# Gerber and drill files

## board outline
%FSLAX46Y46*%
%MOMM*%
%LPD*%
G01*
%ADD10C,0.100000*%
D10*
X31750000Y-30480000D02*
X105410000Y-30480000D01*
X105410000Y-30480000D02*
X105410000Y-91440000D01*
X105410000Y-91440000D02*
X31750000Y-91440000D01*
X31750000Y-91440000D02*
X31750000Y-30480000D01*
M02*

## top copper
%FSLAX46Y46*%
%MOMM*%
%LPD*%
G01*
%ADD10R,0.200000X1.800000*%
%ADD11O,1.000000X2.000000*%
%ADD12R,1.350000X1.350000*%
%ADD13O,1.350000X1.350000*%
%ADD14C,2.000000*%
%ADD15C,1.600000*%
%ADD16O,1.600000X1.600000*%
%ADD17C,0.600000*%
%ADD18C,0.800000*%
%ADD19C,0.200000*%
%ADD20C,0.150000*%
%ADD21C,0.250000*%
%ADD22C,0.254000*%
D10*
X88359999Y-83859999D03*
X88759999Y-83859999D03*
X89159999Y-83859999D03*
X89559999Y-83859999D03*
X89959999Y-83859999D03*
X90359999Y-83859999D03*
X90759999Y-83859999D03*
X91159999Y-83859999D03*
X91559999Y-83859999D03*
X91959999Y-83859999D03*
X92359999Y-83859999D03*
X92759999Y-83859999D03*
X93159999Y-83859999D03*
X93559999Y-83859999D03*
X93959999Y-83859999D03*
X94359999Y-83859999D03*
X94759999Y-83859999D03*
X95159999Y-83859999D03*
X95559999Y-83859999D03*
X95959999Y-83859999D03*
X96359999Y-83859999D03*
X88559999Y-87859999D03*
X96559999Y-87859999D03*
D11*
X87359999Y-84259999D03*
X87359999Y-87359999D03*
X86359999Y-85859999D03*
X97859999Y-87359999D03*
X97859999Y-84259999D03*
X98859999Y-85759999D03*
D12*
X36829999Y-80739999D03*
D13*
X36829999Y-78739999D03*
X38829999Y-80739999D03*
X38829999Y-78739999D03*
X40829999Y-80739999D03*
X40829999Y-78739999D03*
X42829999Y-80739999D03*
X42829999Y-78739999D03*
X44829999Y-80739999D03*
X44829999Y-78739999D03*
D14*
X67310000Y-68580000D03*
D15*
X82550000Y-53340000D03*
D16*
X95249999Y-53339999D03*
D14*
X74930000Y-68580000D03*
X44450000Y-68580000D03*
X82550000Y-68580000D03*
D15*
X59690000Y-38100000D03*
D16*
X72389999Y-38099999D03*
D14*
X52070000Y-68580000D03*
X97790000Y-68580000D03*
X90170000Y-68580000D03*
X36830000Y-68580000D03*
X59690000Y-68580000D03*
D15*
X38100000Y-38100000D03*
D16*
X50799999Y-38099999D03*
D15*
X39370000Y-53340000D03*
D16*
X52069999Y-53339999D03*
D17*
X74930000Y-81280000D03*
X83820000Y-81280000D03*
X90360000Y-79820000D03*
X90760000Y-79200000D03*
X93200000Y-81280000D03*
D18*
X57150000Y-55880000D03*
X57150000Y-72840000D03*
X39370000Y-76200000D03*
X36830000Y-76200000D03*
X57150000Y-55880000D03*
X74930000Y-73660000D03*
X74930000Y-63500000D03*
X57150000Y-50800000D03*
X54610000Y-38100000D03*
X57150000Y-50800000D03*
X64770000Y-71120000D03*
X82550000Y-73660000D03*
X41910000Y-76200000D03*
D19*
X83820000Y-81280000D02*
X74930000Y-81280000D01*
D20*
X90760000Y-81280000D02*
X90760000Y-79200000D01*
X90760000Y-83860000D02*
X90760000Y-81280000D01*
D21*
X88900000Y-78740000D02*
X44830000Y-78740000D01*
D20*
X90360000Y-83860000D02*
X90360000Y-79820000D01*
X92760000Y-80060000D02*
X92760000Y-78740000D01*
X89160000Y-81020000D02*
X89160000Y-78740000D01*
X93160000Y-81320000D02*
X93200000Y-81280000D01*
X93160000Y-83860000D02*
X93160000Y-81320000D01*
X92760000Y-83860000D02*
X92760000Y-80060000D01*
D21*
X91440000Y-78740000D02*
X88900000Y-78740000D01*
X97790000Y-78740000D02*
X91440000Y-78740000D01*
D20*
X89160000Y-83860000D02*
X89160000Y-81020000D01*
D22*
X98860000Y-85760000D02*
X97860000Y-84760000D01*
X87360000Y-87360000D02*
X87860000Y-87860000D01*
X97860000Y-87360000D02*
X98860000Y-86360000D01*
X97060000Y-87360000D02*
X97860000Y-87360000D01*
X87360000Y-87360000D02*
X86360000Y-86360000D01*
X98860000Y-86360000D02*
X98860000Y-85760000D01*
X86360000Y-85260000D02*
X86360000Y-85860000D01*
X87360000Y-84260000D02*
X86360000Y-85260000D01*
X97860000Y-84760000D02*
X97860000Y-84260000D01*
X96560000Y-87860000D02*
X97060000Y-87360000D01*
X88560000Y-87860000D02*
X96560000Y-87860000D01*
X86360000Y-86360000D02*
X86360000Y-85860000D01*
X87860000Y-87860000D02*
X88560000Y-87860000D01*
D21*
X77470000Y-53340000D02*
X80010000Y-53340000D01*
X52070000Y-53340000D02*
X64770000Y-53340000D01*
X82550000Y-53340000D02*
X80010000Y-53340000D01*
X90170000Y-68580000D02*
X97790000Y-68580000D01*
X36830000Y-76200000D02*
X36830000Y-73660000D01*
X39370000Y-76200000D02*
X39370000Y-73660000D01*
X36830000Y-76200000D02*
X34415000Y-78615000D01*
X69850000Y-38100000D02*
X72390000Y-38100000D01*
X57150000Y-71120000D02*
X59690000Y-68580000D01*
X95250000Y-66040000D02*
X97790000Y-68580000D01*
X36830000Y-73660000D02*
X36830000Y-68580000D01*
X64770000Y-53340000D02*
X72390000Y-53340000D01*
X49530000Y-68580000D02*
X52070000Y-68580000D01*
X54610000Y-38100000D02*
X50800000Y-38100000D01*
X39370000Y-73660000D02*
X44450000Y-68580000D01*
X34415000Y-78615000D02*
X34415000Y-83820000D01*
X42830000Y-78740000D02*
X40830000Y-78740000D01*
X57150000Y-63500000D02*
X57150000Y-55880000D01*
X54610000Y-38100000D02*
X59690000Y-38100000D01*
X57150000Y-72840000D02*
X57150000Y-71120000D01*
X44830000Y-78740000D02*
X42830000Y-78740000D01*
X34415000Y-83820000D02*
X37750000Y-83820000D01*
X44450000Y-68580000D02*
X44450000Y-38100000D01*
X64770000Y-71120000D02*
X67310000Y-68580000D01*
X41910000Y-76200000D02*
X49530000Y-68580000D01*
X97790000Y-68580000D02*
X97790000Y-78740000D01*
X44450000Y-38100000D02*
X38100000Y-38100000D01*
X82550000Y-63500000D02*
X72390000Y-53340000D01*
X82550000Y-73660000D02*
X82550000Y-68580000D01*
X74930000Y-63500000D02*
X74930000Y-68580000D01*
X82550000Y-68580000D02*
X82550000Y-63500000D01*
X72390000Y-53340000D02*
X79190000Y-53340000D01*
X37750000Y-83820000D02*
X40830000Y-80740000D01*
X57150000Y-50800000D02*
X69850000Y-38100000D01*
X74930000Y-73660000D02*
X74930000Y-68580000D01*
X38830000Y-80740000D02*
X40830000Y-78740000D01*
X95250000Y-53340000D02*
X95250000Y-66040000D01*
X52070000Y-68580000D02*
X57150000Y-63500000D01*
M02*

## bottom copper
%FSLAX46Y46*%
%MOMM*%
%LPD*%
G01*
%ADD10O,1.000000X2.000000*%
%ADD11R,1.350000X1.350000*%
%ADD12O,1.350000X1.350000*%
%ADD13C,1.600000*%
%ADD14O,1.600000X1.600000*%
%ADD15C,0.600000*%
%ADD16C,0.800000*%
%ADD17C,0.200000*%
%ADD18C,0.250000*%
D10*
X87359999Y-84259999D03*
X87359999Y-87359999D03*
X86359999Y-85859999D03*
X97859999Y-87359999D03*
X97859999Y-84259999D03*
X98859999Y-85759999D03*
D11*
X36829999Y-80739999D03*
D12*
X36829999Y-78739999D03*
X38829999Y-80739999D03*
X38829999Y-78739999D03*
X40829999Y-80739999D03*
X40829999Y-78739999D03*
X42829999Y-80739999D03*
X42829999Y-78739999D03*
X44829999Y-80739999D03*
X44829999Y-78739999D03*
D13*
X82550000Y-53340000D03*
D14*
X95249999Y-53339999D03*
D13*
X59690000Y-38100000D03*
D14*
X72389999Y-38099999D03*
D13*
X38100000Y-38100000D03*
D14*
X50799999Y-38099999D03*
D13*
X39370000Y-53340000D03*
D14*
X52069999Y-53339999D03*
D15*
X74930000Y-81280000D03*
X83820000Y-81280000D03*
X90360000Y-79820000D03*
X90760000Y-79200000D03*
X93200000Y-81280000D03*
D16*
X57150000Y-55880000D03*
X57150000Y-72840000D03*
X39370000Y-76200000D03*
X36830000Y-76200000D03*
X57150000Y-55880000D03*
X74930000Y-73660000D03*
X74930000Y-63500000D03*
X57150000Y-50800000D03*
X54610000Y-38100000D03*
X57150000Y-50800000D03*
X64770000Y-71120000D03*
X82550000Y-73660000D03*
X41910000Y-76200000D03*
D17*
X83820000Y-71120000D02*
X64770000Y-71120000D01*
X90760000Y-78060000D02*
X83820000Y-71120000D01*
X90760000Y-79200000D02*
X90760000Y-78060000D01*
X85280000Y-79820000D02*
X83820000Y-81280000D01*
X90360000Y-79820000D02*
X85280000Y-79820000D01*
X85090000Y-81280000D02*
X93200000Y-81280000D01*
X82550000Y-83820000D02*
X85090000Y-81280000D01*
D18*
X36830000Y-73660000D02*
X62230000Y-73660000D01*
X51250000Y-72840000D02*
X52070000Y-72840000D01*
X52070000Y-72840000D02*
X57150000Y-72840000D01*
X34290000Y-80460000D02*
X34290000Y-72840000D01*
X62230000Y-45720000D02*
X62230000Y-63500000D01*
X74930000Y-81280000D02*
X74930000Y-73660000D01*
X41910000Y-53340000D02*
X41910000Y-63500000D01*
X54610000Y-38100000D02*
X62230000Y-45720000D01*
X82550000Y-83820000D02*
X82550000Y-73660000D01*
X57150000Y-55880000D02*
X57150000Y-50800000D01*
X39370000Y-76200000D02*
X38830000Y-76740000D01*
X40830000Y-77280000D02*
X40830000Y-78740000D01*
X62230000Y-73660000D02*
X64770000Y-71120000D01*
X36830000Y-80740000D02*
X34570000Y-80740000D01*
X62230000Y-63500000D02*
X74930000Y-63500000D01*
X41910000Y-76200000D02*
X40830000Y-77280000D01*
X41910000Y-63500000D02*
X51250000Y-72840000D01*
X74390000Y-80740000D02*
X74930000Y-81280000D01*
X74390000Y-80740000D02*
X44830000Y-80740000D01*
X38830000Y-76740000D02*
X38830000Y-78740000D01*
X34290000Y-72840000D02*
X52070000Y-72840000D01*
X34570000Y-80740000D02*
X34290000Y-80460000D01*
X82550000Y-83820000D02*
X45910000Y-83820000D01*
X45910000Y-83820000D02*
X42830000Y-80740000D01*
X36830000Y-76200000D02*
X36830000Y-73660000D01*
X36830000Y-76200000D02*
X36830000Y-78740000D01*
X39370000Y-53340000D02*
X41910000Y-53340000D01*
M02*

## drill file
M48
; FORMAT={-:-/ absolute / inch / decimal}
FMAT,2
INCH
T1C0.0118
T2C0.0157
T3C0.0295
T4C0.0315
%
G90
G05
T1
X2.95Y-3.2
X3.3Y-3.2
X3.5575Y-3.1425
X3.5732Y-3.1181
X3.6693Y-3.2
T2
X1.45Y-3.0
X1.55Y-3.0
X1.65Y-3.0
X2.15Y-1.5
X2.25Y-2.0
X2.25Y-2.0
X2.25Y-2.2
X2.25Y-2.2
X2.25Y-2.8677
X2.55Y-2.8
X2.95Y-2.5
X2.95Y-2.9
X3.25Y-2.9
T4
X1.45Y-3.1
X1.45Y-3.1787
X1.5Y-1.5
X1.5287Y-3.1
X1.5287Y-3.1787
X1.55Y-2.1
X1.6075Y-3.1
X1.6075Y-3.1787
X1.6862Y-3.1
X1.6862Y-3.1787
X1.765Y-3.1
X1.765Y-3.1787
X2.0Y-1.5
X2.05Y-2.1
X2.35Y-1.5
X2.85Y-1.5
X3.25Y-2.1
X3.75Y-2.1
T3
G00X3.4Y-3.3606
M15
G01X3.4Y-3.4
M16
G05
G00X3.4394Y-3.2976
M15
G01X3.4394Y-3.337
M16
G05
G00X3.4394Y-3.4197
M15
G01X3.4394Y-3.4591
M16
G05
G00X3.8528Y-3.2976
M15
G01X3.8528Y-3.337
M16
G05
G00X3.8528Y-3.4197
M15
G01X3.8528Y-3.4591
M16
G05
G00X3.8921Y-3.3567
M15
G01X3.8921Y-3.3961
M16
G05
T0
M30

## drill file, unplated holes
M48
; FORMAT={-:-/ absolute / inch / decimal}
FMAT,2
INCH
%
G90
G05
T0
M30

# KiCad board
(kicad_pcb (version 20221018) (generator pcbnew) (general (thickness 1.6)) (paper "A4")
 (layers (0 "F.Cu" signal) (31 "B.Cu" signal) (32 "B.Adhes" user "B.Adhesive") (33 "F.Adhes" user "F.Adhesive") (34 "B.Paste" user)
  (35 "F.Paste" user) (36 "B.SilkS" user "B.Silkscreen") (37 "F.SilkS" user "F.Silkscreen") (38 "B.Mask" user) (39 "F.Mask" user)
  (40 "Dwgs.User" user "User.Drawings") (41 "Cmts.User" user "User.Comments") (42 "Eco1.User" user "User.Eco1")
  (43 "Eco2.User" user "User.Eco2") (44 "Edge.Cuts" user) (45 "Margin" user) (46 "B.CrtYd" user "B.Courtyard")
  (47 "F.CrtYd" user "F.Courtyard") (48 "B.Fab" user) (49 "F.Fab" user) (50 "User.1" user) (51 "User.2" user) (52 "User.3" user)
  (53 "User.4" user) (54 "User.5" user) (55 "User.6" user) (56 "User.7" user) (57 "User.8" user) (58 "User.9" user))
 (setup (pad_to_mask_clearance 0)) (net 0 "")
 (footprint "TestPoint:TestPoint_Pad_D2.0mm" (layer "F.Cu") (at 67.31 68.58)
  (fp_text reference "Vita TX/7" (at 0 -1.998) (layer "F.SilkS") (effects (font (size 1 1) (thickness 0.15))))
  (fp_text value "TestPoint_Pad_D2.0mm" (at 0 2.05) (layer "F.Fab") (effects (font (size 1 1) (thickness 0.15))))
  (pad "1" smd circle (at 0 0) (size 2 2) (layers "F.Cu" "F.Mask")))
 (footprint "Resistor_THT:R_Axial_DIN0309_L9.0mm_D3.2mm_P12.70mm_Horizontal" (layer "F.Cu") (at 59.69 38.1)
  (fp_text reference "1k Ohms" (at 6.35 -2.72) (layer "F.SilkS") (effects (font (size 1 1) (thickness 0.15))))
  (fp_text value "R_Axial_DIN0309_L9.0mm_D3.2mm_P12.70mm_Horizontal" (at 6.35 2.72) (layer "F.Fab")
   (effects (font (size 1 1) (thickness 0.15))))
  (pad "1" thru_hole circle (at 0 0) (size 1.6 1.6) (drill 0.8) (layers "*.Cu" "*.Mask"))
  (pad "2" thru_hole oval (at 12.7 0) (size 1.6 1.6) (drill 0.8) (layers "*.Cu" "*.Mask")))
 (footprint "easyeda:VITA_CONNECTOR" (layer "F.Cu") (at 87.36 84.26)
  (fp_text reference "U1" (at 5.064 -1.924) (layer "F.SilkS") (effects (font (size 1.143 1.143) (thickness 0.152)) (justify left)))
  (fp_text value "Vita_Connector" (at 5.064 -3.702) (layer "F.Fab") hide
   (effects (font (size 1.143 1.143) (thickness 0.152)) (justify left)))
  (pad "1" smd rect (at 1 -0.4) (size 0.2 1.8) (layers "F.Cu" "F.Paste" "F.Mask"))
  (pad "2" smd rect (at 1.4 -0.4) (size 0.2 1.8) (layers "F.Cu" "F.Paste" "F.Mask"))
  (pad "3" smd rect (at 1.8 -0.4) (size 0.2 1.8) (layers "F.Cu" "F.Paste" "F.Mask"))
  (pad "4" smd rect (at 2.2 -0.4) (size 0.2 1.8) (layers "F.Cu" "F.Paste" "F.Mask"))
  (pad "5" smd rect (at 2.6 -0.4) (size 0.2 1.8) (layers "F.Cu" "F.Paste" "F.Mask"))
  (pad "6" smd rect (at 3 -0.4) (size 0.2 1.8) (layers "F.Cu" "F.Paste" "F.Mask"))
  (pad "7" smd rect (at 3.4 -0.4) (size 0.2 1.8) (layers "F.Cu" "F.Paste" "F.Mask"))
  (pad "8" smd rect (at 3.8 -0.4) (size 0.2 1.8) (layers "F.Cu" "F.Paste" "F.Mask"))
  (pad "9" smd rect (at 4.2 -0.4) (size 0.2 1.8) (layers "F.Cu" "F.Paste" "F.Mask"))
  (pad "10" smd rect (at 4.6 -0.4) (size 0.2 1.8) (layers "F.Cu" "F.Paste" "F.Mask"))
  (pad "11" smd rect (at 5 -0.4) (size 0.2 1.8) (layers "F.Cu" "F.Paste" "F.Mask"))
  (pad "12" smd rect (at 5.4 -0.4) (size 0.2 1.8) (layers "F.Cu" "F.Paste" "F.Mask"))
  (pad "13" smd rect (at 5.8 -0.4) (size 0.2 1.8) (layers "F.Cu" "F.Paste" "F.Mask"))
  (pad "14" smd rect (at 6.2 -0.4) (size 0.2 1.8) (layers "F.Cu" "F.Paste" "F.Mask"))
  (pad "15" smd rect (at 6.6 -0.4) (size 0.2 1.8) (layers "F.Cu" "F.Paste" "F.Mask"))
  (pad "16" smd rect (at 7 -0.4) (size 0.2 1.8) (layers "F.Cu" "F.Paste" "F.Mask"))
  (pad "17" smd rect (at 7.4 -0.4) (size 0.2 1.8) (layers "F.Cu" "F.Paste" "F.Mask"))
  (pad "18" smd rect (at 7.8 -0.4) (size 0.2 1.8) (layers "F.Cu" "F.Paste" "F.Mask"))
  (pad "19" smd rect (at 8.2 -0.4) (size 0.2 1.8) (layers "F.Cu" "F.Paste" "F.Mask"))
  (pad "20" smd rect (at 8.6 -0.4) (size 0.2 1.8) (layers "F.Cu" "F.Paste" "F.Mask"))
  (pad "21" smd rect (at 9 -0.4) (size 0.2 1.8) (layers "F.Cu" "F.Paste" "F.Mask"))
  (pad "22" smd rect (at 1.2 3.6) (size 0.2 1.8) (layers "F.Cu" "F.Paste" "F.Mask"))
  (pad "23" smd rect (at 9.2 3.6) (size 0.2 1.8) (layers "F.Cu" "F.Paste" "F.Mask"))
  (pad "24" thru_hole oval (at 0 0) (size 1 2) (drill oval 0.75 1.75) (layers "*.Cu" "*.Paste" "*.Mask"))
  (pad "25" thru_hole oval (at 0 3.1) (size 1 2) (drill oval 0.75 1.75) (layers "*.Cu" "*.Paste" "*.Mask"))
  (pad "26" thru_hole oval (at -1 1.6) (size 1 2) (drill oval 0.75 1.75) (layers "*.Cu" "*.Paste" "*.Mask"))
  (pad "27" thru_hole oval (at 10.5 3.1) (size 1 2) (drill oval 0.75 1.75) (layers "*.Cu" "*.Paste" "*.Mask"))
  (pad "28" thru_hole oval (at 10.5 0) (size 1 2) (drill oval 0.75 1.75) (layers "*.Cu" "*.Paste" "*.Mask"))
  (pad "29" thru_hole oval (at 11.5 1.5) (size 1 2) (drill oval 0.75 1.75) (layers "*.Cu" "*.Paste" "*.Mask")))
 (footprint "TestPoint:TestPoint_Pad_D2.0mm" (layer "F.Cu") (at 44.45 68.58)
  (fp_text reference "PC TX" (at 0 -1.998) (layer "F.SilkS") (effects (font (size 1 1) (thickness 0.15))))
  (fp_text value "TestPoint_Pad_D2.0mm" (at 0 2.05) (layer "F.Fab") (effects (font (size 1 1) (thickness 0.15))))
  (pad "1" smd circle (at 0 0) (size 2 2) (layers "F.Cu" "F.Mask")))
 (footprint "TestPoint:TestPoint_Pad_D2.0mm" (layer "F.Cu") (at 90.17 68.58)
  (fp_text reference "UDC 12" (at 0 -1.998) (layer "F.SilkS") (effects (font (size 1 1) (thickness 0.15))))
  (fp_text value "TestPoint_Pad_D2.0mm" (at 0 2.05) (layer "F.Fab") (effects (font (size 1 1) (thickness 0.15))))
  (pad "1" smd circle (at 0 0) (size 2 2) (layers "F.Cu" "F.Mask")))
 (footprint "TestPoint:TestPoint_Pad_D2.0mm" (layer "F.Cu") (at 82.55 68.58)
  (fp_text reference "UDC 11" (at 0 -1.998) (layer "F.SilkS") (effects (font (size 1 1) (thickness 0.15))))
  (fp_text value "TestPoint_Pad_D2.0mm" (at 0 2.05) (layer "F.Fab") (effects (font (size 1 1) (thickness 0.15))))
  (pad "1" smd circle (at 0 0) (size 2 2) (layers "F.Cu" "F.Mask")))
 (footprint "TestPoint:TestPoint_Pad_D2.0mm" (layer "F.Cu") (at 74.93 68.58)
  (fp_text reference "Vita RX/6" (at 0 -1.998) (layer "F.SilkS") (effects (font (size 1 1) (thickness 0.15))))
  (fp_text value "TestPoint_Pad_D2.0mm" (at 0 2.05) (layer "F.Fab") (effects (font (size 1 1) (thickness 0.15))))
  (pad "1" smd circle (at 0 0) (size 2 2) (layers "F.Cu" "F.Mask")))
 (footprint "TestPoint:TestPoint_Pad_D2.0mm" (layer "F.Cu") (at 36.83 68.58)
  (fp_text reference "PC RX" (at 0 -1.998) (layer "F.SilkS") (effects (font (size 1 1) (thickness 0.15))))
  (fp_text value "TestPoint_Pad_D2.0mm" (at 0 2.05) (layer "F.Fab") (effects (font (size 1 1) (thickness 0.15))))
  (pad "1" smd circle (at 0 0) (size 2 2) (layers "F.Cu" "F.Mask")))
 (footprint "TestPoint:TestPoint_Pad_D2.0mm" (layer "F.Cu") (at 97.79 68.58)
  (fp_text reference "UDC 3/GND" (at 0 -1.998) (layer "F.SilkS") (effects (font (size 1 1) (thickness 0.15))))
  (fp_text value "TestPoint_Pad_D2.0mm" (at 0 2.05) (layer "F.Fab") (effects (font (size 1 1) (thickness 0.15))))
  (pad "1" smd circle (at 0 0) (size 2 2) (layers "F.Cu" "F.Mask")))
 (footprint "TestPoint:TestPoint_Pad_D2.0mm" (layer "F.Cu") (at 59.69 68.58)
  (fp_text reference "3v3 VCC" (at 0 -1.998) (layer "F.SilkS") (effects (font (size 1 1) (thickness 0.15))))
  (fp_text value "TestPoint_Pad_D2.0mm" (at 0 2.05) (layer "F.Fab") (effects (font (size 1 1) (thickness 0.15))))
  (pad "1" smd circle (at 0 0) (size 2 2) (layers "F.Cu" "F.Mask")))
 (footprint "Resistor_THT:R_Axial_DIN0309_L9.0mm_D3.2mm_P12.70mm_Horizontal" (layer "F.Cu") (at 82.55 53.34)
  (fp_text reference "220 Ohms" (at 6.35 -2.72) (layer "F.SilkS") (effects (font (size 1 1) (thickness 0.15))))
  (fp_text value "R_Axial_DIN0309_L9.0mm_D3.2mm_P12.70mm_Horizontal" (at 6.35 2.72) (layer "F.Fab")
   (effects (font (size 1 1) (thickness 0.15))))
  (pad "1" thru_hole circle (at 0 0) (size 1.6 1.6) (drill 0.8) (layers "*.Cu" "*.Mask"))
  (pad "2" thru_hole oval (at 12.7 0) (size 1.6 1.6) (drill 0.8) (layers "*.Cu" "*.Mask")))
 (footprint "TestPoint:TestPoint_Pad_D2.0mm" (layer "F.Cu") (at 52.07 68.58)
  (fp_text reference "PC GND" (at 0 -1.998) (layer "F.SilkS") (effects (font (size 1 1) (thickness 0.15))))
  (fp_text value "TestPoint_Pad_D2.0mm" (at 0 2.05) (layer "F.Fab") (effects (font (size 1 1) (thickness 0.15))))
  (pad "1" smd circle (at 0 0) (size 2 2) (layers "F.Cu" "F.Mask")))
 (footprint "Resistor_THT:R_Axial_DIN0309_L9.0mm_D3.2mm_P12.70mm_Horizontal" (layer "F.Cu") (at 39.37 53.34)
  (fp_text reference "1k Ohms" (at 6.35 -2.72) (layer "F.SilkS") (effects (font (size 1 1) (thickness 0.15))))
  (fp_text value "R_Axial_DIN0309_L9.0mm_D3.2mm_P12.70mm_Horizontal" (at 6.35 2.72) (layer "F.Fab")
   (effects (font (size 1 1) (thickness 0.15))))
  (pad "1" thru_hole circle (at 0 0) (size 1.6 1.6) (drill 0.8) (layers "*.Cu" "*.Mask"))
  (pad "2" thru_hole oval (at 12.7 0) (size 1.6 1.6) (drill 0.8) (layers "*.Cu" "*.Mask")))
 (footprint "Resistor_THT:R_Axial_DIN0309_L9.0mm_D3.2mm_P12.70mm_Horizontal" (layer "F.Cu") (at 38.1 38.1)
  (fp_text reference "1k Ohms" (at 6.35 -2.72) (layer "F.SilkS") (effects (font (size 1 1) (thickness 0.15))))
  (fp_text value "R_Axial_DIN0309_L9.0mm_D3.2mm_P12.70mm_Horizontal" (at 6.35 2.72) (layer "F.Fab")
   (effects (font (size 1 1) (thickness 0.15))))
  (pad "1" thru_hole circle (at 0 0) (size 1.6 1.6) (drill 0.8) (layers "*.Cu" "*.Mask"))
  (pad "2" thru_hole oval (at 12.7 0) (size 1.6 1.6) (drill 0.8) (layers "*.Cu" "*.Mask")))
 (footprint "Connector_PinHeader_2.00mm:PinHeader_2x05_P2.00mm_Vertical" (layer "F.Cu") (at 36.83 80.74 90)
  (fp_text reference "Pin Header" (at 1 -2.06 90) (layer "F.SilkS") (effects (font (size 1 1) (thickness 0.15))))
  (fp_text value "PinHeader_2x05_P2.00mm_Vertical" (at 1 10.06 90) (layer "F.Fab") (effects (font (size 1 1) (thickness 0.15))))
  (pad "1" thru_hole rect (at 0 0 90) (size 1.35 1.35) (drill 0.8) (layers "*.Cu" "*.Mask"))
  (pad "2" thru_hole oval (at 2 0 90) (size 1.35 1.35) (drill 0.8) (layers "*.Cu" "*.Mask"))
  (pad "3" thru_hole oval (at 0 2 90) (size 1.35 1.35) (drill 0.8) (layers "*.Cu" "*.Mask"))
  (pad "4" thru_hole oval (at 2 2 90) (size 1.35 1.35) (drill 0.8) (layers "*.Cu" "*.Mask"))
  (pad "5" thru_hole oval (at 0 4 90) (size 1.35 1.35) (drill 0.8) (layers "*.Cu" "*.Mask"))
  (pad "6" thru_hole oval (at 2 4 90) (size 1.35 1.35) (drill 0.8) (layers "*.Cu" "*.Mask"))
  (pad "7" thru_hole oval (at 0 6 90) (size 1.35 1.35) (drill 0.8) (layers "*.Cu" "*.Mask"))
  (pad "8" thru_hole oval (at 2 6 90) (size 1.35 1.35) (drill 0.8) (layers "*.Cu" "*.Mask"))
  (pad "9" thru_hole oval (at 0 8 90) (size 1.35 1.35) (drill 0.8) (layers "*.Cu" "*.Mask"))
  (pad "10" thru_hole oval (at 2 8 90) (size 1.35 1.35) (drill 0.8) (layers "*.Cu" "*.Mask")))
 (gr_rect (start 31.75 30.48) (end 105.41 91.44) (stroke (width 0.1) (type default)) (fill none) (layer "Edge.Cuts"))
 (segment (start 82.55 53.34) (end 80.01 53.34) (width 0.25) (layer "F.Cu") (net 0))
 (segment (start 88.9 78.74) (end 44.83 78.74) (width 0.25) (layer "F.Cu") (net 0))
 (segment (start 72.39 53.34) (end 79.19 53.34) (width 0.25) (layer "F.Cu") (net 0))
 (segment (start 69.85 38.1) (end 72.39 38.1) (width 0.25) (layer "F.Cu") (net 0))
 (segment (start 95.25 53.34) (end 95.25 66.04) (width 0.25) (layer "F.Cu") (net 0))
 (segment (start 89.16 81.02) (end 89.16 78.74) (width 0.15) (layer "F.Cu") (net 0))
 (segment (start 97.79 78.74) (end 91.44 78.74) (width 0.25) (layer "F.Cu") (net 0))
 (segment (start 86.36 86.36) (end 86.36 85.86) (width 0.254) (layer "F.Cu") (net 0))
 (segment (start 96.56 87.86) (end 97.06 87.36) (width 0.254) (layer "F.Cu") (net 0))
 (segment (start 87.36 87.36) (end 86.36 86.36) (width 0.254) (layer "F.Cu") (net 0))
 (segment (start 86.36 85.26) (end 86.36 85.86) (width 0.254) (layer "F.Cu") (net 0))
 (segment (start 87.36 87.36) (end 87.86 87.86) (width 0.254) (layer "F.Cu") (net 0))
 (segment (start 95.25 66.04) (end 97.79 68.58) (width 0.25) (layer "F.Cu") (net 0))
 (segment (start 74.93 73.66) (end 74.93 68.58) (width 0.25) (layer "F.Cu") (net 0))
 (segment (start 54.61 38.1) (end 59.69 38.1) (width 0.25) (layer "F.Cu") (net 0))
 (segment (start 83.82 81.28) (end 74.93 81.28) (width 0.2) (layer "F.Cu") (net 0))
 (segment (start 44.45 68.58) (end 44.45 38.1) (width 0.25) (layer "F.Cu") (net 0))
 (segment (start 97.79 68.58) (end 97.79 78.74) (width 0.25) (layer "F.Cu") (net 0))
 (segment (start 90.36 83.86) (end 90.36 79.82) (width 0.15) (layer "F.Cu") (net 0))
 (segment (start 87.86 87.86) (end 88.56 87.86) (width 0.254) (layer "F.Cu") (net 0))
 (segment (start 82.55 68.58) (end 82.55 63.5) (width 0.25) (layer "F.Cu") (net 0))
 (segment (start 98.86 85.76) (end 97.86 84.76) (width 0.254) (layer "F.Cu") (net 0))
 (segment (start 52.07 68.58) (end 57.15 63.5) (width 0.25) (layer "F.Cu") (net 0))
 (segment (start 64.77 53.34) (end 72.39 53.34) (width 0.25) (layer "F.Cu") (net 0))
 (segment (start 34.415 83.82) (end 37.75 83.82) (width 0.25) (layer "F.Cu") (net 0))
 (segment (start 93.16 81.32) (end 93.2 81.28) (width 0.15) (layer "F.Cu") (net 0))
 (segment (start 49.53 68.58) (end 52.07 68.58) (width 0.25) (layer "F.Cu") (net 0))
 (segment (start 57.15 71.12) (end 59.69 68.58) (width 0.25) (layer "F.Cu") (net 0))
 (segment (start 82.55 63.5) (end 72.39 53.34) (width 0.25) (layer "F.Cu") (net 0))
 (segment (start 34.415 78.615) (end 34.415 83.82) (width 0.25) (layer "F.Cu") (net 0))
 (segment (start 38.83 80.74) (end 40.83 78.74) (width 0.25) (layer "F.Cu") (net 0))
 (segment (start 36.83 76.2) (end 34.415 78.615) (width 0.25) (layer "F.Cu") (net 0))
 (segment (start 36.83 73.66) (end 36.83 68.58) (width 0.25) (layer "F.Cu") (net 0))
 (segment (start 57.15 63.5) (end 57.15 55.88) (width 0.25) (layer "F.Cu") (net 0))
 (segment (start 82.55 73.66) (end 82.55 68.58) (width 0.25) (layer "F.Cu") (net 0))
 (segment (start 90.17 68.58) (end 97.79 68.58) (width 0.25) (layer "F.Cu") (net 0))
 (segment (start 97.86 84.76) (end 97.86 84.26) (width 0.254) (layer "F.Cu") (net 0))
 (segment (start 93.16 83.86) (end 93.16 81.32) (width 0.15) (layer "F.Cu") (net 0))
 (segment (start 41.91 76.2) (end 49.53 68.58) (width 0.25) (layer "F.Cu") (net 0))
 (segment (start 44.45 38.1) (end 38.1 38.1) (width 0.25) (layer "F.Cu") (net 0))
 (segment (start 37.75 83.82) (end 40.83 80.74) (width 0.25) (layer "F.Cu") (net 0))
 (segment (start 98.86 86.36) (end 98.86 85.76) (width 0.254) (layer "F.Cu") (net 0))
 (segment (start 74.93 63.5) (end 74.93 68.58) (width 0.25) (layer "F.Cu") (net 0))
 (segment (start 92.76 80.06) (end 92.76 78.74) (width 0.15) (layer "F.Cu") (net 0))
 (segment (start 39.37 73.66) (end 44.45 68.58) (width 0.25) (layer "F.Cu") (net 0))
 (segment (start 57.15 72.84) (end 57.15 71.12) (width 0.25) (layer "F.Cu") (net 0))
 (segment (start 87.36 84.26) (end 86.36 85.26) (width 0.254) (layer "F.Cu") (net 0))
 (segment (start 36.83 76.2) (end 36.83 73.66) (width 0.25) (layer "F.Cu") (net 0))
 (segment (start 88.56 87.86) (end 96.56 87.86) (width 0.254) (layer "F.Cu") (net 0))
 (segment (start 77.47 53.34) (end 80.01 53.34) (width 0.25) (layer "F.Cu") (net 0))
 (segment (start 64.77 71.12) (end 67.31 68.58) (width 0.25) (layer "F.Cu") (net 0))
 (segment (start 91.44 78.74) (end 88.9 78.74) (width 0.25) (layer "F.Cu") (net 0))
 (segment (start 42.83 78.74) (end 40.83 78.74) (width 0.25) (layer "F.Cu") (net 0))
 (segment (start 92.76 83.86) (end 92.76 80.06) (width 0.15) (layer "F.Cu") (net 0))
 (segment (start 54.61 38.1) (end 50.8 38.1) (width 0.25) (layer "F.Cu") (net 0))
 (segment (start 52.07 53.34) (end 64.77 53.34) (width 0.25) (layer "F.Cu") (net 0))
 (segment (start 39.37 76.2) (end 39.37 73.66) (width 0.25) (layer "F.Cu") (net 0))
 (segment (start 89.16 83.86) (end 89.16 81.02) (width 0.15) (layer "F.Cu") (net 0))
 (segment (start 44.83 78.74) (end 42.83 78.74) (width 0.25) (layer "F.Cu") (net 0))
 (segment (start 90.76 83.86) (end 90.76 81.28) (width 0.15) (layer "F.Cu") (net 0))
 (segment (start 57.15 50.8) (end 69.85 38.1) (width 0.25) (layer "F.Cu") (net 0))
 (segment (start 97.06 87.36) (end 97.86 87.36) (width 0.254) (layer "F.Cu") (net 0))
 (segment (start 97.86 87.36) (end 98.86 86.36) (width 0.254) (layer "F.Cu") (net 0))
 (segment (start 90.76 81.28) (end 90.76 79.2) (width 0.15) (layer "F.Cu") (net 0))
 (via (at 82.55 73.66) (size 0.8) (drill 0.4) (layers "F.Cu" "B.Cu") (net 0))
 (via (at 74.93 81.28) (size 0.6) (drill 0.3) (layers "F.Cu" "B.Cu") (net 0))
 (via (at 54.61 38.1) (size 0.8) (drill 0.4) (layers "F.Cu" "B.Cu") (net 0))
 (via (at 74.93 73.66) (size 0.8) (drill 0.4) (layers "F.Cu" "B.Cu") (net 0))
 (via (at 57.15 72.84) (size 0.8) (drill 0.4) (layers "F.Cu" "B.Cu") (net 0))
 (via (at 90.36 79.82) (size 0.6) (drill 0.3) (layers "F.Cu" "B.Cu") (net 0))
 (via (at 93.2 81.28) (size 0.6) (drill 0.3) (layers "F.Cu" "B.Cu") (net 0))
 (via (at 57.15 55.88) (size 0.8) (drill 0.4) (layers "F.Cu" "B.Cu") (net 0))
 (via (at 90.76 79.2) (size 0.6) (drill 0.3) (layers "F.Cu" "B.Cu") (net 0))
 (via (at 57.15 50.8) (size 0.8) (drill 0.4) (layers "F.Cu" "B.Cu") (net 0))
 (via (at 83.82 81.28) (size 0.6) (drill 0.3) (layers "F.Cu" "B.Cu") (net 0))
 (via (at 39.37 76.2) (size 0.8) (drill 0.4) (layers "F.Cu" "B.Cu") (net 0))
 (via (at 36.83 76.2) (size 0.8) (drill 0.4) (layers "F.Cu" "B.Cu") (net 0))
 (via (at 57.15 50.8) (size 0.8) (drill 0.4) (layers "F.Cu" "B.Cu") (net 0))
 (via (at 57.15 55.88) (size 0.8) (drill 0.4) (layers "F.Cu" "B.Cu") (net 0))
 (via (at 41.91 76.2) (size 0.8) (drill 0.4) (layers "F.Cu" "B.Cu") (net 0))
 (via (at 64.77 71.12) (size 0.8) (drill 0.4) (layers "F.Cu" "B.Cu") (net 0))
 (via (at 74.93 63.5) (size 0.8) (drill 0.4) (layers "F.Cu" "B.Cu") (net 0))
 (segment (start 82.55 83.82) (end 85.09 81.28) (width 0.2) (layer "B.Cu") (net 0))
 (segment (start 45.91 83.82) (end 42.83 80.74) (width 0.25) (layer "B.Cu") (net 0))
 (segment (start 52.07 72.84) (end 57.15 72.84) (width 0.25) (layer "B.Cu") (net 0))
 (segment (start 40.83 77.28) (end 40.83 78.74) (width 0.25) (layer "B.Cu") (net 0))
 (segment (start 36.83 76.2) (end 36.83 78.74) (width 0.25) (layer "B.Cu") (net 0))
 (segment (start 38.83 76.74) (end 38.83 78.74) (width 0.25) (layer "B.Cu") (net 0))
 (segment (start 36.83 76.2) (end 36.83 73.66) (width 0.25) (layer "B.Cu") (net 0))
 (segment (start 54.61 38.1) (end 62.23 45.72) (width 0.25) (layer "B.Cu") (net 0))
 (segment (start 39.37 76.2) (end 38.83 76.74) (width 0.25) (layer "B.Cu") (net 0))
 (segment (start 51.25 72.84) (end 52.07 72.84) (width 0.25) (layer "B.Cu") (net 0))
 (segment (start 62.23 63.5) (end 74.93 63.5) (width 0.25) (layer "B.Cu") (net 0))
 (segment (start 57.15 55.88) (end 57.15 50.8) (width 0.25) (layer "B.Cu") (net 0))
 (segment (start 74.39 80.74) (end 44.83 80.74) (width 0.25) (layer "B.Cu") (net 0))
 (segment (start 90.76 78.06) (end 83.82 71.12) (width 0.2) (layer "B.Cu") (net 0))
 (segment (start 90.36 79.82) (end 85.28 79.82) (width 0.2) (layer "B.Cu") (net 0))
 (segment (start 74.93 81.28) (end 74.93 73.66) (width 0.25) (layer "B.Cu") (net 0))
 (segment (start 41.91 76.2) (end 40.83 77.28) (width 0.25) (layer "B.Cu") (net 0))
 (segment (start 85.28 79.82) (end 83.82 81.28) (width 0.2) (layer "B.Cu") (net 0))
 (segment (start 90.76 79.2) (end 90.76 78.06) (width 0.2) (layer "B.Cu") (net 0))
 (segment (start 74.39 80.74) (end 74.93 81.28) (width 0.25) (layer "B.Cu") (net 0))
 (segment (start 36.83 73.66) (end 62.23 73.66) (width 0.25) (layer "B.Cu") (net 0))
 (segment (start 39.37 53.34) (end 41.91 53.34) (width 0.25) (layer "B.Cu") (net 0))
 (segment (start 62.23 45.72) (end 62.23 63.5) (width 0.25) (layer "B.Cu") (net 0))
 (segment (start 34.29 72.84) (end 52.07 72.84) (width 0.25) (layer "B.Cu") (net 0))
 (segment (start 85.09 81.28) (end 93.2 81.28) (width 0.2) (layer "B.Cu") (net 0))
 (segment (start 82.55 83.82) (end 45.91 83.82) (width 0.25) (layer "B.Cu") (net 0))
 (segment (start 62.23 73.66) (end 64.77 71.12) (width 0.25) (layer "B.Cu") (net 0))
 (segment (start 34.57 80.74) (end 34.29 80.46) (width 0.25) (layer "B.Cu") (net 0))
 (segment (start 41.91 63.5) (end 51.25 72.84) (width 0.25) (layer "B.Cu") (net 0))
 (segment (start 41.91 53.34) (end 41.91 63.5) (width 0.25) (layer "B.Cu") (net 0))
 (segment (start 82.55 83.82) (end 82.55 73.66) (width 0.25) (layer "B.Cu") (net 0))
 (segment (start 83.82 71.12) (end 64.77 71.12) (width 0.2) (layer "B.Cu") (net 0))
 (segment (start 34.29 80.46) (end 34.29 72.84) (width 0.25) (layer "B.Cu") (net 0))
 (segment (start 36.83 80.74) (end 34.57 80.74) (width 0.25) (layer "B.Cu") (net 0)))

